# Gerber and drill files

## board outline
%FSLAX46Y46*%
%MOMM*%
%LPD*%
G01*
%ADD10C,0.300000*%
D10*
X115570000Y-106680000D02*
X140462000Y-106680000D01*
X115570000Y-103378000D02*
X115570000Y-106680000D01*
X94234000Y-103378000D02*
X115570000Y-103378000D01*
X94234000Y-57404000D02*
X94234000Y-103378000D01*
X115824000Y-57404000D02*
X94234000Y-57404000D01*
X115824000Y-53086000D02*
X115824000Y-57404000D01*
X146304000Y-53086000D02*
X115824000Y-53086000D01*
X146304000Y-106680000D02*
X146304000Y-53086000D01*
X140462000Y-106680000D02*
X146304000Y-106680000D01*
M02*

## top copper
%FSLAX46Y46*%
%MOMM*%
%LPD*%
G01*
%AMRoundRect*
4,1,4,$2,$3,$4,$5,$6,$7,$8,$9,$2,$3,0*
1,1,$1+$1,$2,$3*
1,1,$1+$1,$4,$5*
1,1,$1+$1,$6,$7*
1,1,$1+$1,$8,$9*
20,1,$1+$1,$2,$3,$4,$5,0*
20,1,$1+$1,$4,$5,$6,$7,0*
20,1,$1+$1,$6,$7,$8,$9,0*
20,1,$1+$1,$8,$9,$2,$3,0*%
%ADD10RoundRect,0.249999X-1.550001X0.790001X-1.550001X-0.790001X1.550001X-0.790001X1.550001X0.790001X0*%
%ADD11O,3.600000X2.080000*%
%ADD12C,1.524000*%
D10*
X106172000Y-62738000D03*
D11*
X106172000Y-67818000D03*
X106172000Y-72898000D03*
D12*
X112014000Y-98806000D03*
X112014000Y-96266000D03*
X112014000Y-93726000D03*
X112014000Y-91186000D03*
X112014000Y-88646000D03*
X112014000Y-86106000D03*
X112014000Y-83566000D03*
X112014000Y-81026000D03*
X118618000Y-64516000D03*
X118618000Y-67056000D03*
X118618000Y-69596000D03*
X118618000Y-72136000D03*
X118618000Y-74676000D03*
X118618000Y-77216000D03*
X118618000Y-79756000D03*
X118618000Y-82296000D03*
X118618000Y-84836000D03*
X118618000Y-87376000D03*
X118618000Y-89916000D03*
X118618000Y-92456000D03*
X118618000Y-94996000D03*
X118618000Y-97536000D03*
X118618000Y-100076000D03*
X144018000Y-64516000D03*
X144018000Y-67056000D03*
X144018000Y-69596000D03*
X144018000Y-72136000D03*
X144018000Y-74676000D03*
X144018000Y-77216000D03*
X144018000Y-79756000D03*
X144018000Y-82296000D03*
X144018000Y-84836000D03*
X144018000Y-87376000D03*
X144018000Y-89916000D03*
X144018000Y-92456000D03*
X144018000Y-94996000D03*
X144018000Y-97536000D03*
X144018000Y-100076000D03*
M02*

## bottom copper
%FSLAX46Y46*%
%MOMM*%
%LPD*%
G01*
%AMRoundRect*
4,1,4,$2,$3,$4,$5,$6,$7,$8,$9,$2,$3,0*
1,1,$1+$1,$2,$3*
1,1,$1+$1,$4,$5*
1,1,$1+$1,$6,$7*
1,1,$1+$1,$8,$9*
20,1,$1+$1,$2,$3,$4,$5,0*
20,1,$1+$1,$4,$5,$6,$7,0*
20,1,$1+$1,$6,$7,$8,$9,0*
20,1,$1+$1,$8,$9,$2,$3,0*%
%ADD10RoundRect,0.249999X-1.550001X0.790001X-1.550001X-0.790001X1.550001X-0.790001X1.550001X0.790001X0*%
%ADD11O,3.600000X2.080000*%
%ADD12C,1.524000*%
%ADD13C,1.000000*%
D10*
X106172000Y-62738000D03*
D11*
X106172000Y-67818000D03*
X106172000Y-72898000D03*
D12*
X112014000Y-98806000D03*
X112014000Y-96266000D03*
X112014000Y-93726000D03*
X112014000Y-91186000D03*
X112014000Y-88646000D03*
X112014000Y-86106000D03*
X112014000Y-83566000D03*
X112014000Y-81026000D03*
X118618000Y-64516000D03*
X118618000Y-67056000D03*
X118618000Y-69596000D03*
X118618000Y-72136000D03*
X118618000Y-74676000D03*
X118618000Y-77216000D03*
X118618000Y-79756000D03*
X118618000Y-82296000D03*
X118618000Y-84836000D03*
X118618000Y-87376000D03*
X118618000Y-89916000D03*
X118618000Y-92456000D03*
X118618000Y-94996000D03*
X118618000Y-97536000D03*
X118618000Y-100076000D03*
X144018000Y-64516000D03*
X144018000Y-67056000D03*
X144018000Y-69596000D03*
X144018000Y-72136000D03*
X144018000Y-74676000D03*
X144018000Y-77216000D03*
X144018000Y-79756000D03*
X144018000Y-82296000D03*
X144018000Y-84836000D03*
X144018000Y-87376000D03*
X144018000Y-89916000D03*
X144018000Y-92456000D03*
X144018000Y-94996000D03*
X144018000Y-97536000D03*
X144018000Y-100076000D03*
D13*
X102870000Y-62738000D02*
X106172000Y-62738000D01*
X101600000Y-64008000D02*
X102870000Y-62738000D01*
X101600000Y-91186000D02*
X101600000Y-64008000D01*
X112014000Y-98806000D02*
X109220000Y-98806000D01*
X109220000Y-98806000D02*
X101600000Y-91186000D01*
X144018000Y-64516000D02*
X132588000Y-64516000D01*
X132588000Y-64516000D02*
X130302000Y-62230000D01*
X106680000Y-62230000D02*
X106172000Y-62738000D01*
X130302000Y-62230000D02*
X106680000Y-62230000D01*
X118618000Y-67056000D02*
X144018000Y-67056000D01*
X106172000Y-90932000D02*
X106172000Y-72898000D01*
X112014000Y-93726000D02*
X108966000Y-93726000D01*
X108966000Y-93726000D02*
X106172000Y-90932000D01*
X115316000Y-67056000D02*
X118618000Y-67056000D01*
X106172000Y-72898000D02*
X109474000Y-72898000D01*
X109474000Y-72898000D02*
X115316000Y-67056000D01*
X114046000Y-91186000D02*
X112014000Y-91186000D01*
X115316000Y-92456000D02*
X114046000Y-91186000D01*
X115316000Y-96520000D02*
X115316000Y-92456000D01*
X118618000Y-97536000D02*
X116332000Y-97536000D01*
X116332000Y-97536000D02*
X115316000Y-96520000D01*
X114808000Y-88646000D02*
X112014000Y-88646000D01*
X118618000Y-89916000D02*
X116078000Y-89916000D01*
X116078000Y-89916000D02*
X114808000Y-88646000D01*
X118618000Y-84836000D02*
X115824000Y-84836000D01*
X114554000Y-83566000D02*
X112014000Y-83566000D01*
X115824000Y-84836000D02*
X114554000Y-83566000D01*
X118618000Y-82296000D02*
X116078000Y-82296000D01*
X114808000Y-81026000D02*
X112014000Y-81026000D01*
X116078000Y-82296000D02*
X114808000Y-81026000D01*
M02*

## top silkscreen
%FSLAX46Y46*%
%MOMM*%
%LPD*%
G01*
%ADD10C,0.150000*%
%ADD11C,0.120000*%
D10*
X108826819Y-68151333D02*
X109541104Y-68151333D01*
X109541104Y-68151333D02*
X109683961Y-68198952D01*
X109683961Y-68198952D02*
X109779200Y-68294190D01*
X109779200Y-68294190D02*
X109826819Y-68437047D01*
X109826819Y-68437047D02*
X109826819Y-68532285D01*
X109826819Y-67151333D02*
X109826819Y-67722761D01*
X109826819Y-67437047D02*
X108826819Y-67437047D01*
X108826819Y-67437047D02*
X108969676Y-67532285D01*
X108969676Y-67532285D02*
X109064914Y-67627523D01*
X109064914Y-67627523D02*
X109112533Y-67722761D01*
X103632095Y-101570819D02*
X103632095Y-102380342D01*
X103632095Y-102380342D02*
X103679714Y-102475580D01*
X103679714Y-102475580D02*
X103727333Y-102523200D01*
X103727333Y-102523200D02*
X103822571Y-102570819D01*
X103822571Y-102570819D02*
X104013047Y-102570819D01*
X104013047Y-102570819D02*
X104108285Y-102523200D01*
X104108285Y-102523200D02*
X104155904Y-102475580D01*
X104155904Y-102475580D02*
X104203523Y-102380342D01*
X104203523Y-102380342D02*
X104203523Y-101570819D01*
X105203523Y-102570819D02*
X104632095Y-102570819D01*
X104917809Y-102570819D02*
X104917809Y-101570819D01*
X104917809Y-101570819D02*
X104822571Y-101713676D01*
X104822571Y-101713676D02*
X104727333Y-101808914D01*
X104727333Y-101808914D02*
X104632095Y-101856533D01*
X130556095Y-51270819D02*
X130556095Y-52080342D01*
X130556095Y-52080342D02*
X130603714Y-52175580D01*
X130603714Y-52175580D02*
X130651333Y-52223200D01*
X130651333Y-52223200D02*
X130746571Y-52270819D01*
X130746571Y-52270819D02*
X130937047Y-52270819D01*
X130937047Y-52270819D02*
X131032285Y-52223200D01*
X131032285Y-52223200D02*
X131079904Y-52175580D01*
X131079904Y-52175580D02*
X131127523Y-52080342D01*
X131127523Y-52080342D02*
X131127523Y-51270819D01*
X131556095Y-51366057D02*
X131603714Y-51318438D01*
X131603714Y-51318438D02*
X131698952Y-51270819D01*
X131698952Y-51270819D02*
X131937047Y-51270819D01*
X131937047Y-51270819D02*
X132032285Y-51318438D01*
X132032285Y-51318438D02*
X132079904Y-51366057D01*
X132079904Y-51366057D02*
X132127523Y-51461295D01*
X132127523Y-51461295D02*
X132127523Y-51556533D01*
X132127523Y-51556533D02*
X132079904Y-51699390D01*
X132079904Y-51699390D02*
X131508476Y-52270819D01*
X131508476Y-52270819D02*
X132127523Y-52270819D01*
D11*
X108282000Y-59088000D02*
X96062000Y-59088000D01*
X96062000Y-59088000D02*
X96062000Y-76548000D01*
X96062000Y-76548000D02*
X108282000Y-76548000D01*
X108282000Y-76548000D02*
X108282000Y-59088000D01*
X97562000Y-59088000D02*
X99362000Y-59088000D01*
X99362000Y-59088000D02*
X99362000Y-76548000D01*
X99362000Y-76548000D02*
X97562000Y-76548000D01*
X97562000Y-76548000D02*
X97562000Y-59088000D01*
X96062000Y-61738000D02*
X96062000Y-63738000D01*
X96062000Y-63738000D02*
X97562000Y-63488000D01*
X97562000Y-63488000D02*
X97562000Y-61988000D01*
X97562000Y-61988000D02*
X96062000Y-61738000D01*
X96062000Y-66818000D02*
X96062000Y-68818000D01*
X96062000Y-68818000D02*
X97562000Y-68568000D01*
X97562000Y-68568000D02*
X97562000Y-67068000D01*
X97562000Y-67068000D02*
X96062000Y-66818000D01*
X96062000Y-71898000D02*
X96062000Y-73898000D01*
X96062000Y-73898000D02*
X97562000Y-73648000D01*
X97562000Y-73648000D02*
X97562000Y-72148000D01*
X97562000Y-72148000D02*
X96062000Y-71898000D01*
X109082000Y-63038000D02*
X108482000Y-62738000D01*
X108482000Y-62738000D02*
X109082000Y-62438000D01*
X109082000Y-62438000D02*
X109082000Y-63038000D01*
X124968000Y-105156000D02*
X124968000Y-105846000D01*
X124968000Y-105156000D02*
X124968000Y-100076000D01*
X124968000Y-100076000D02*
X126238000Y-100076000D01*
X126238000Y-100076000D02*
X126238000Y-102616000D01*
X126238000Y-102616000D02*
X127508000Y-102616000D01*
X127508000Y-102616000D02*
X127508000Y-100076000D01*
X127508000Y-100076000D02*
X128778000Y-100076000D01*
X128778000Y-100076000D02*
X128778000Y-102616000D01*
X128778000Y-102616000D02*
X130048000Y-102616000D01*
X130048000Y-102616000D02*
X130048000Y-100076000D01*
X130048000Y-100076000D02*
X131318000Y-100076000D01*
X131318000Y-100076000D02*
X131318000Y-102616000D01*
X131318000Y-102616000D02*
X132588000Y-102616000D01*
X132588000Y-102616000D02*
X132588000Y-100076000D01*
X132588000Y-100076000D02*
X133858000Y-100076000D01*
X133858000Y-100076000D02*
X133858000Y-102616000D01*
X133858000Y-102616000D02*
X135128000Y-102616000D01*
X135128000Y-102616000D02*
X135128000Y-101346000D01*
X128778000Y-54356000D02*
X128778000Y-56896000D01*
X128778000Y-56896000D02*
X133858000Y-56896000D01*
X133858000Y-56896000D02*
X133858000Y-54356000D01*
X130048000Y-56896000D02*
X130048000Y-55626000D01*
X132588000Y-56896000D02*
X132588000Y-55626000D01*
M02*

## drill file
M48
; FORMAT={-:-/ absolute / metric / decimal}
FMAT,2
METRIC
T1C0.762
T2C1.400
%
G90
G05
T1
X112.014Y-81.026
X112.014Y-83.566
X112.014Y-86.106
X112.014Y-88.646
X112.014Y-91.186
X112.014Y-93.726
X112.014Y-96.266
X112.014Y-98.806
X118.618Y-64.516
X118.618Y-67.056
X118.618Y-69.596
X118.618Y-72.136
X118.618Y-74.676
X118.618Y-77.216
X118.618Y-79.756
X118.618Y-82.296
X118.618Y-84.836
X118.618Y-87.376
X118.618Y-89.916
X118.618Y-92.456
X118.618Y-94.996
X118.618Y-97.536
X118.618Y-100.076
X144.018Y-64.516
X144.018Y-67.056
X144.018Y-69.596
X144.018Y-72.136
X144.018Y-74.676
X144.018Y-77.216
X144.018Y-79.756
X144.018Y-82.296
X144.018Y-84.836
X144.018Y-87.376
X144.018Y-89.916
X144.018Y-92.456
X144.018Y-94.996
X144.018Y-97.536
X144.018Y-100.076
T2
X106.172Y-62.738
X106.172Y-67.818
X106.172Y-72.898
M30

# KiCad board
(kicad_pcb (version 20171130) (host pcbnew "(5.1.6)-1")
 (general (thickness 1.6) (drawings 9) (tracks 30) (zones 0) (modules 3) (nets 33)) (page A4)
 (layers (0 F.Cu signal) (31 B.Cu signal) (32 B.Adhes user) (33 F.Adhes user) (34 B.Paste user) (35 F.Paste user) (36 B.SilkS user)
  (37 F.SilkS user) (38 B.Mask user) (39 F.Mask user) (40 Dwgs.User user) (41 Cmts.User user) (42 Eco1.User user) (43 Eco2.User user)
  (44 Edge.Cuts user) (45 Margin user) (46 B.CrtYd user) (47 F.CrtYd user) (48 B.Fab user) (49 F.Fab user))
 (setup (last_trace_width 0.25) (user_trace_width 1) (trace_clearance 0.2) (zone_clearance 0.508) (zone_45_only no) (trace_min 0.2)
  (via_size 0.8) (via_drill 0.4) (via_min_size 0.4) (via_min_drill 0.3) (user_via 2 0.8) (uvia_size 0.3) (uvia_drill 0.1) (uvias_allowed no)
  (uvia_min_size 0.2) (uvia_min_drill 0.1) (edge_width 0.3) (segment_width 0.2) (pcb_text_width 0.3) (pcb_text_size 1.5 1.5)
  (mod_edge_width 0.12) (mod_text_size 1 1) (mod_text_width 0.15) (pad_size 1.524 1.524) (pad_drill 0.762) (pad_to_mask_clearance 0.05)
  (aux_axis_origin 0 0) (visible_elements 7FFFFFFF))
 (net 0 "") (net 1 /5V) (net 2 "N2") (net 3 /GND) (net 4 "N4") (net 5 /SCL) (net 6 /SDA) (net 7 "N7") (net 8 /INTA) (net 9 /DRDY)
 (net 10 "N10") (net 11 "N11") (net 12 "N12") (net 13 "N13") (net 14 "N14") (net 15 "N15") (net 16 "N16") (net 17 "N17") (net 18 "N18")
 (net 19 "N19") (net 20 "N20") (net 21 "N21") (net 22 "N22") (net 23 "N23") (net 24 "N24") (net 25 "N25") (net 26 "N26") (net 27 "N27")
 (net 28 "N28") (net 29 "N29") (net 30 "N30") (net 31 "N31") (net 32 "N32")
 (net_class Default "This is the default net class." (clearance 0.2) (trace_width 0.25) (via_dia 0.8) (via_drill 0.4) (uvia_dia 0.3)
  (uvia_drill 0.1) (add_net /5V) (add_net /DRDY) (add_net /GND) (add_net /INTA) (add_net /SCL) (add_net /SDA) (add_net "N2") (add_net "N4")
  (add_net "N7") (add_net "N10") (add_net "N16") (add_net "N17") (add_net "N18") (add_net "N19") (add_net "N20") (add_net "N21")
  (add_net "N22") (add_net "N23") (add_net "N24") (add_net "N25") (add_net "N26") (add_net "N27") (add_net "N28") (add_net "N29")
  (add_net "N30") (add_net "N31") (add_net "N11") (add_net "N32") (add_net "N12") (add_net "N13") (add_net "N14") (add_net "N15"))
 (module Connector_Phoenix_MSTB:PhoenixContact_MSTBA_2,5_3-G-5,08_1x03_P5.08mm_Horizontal (layer F.Cu) (at 106.172 62.738 270)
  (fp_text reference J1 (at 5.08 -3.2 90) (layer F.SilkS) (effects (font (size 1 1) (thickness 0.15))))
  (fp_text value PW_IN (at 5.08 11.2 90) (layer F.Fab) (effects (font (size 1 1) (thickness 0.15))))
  (fp_line (start -3.65 -2.11) (end -3.65 10.11) (layer F.SilkS) (width 0.12))
  (fp_line (start -3.65 10.11) (end 13.81 10.11) (layer F.SilkS) (width 0.12))
  (fp_line (start 13.81 10.11) (end 13.81 -2.11) (layer F.SilkS) (width 0.12))
  (fp_line (start 13.81 -2.11) (end -3.65 -2.11) (layer F.SilkS) (width 0.12))
  (fp_line (start -3.65 8.61) (end -3.65 6.81) (layer F.SilkS) (width 0.12))
  (fp_line (start -3.65 6.81) (end 13.81 6.81) (layer F.SilkS) (width 0.12))
  (fp_line (start 13.81 6.81) (end 13.81 8.61) (layer F.SilkS) (width 0.12))
  (fp_line (start 13.81 8.61) (end -3.65 8.61) (layer F.SilkS) (width 0.12))
  (fp_line (start -1 10.11) (end 1 10.11) (layer F.SilkS) (width 0.12))
  (fp_line (start 1 10.11) (end 0.75 8.61) (layer F.SilkS) (width 0.12))
  (fp_line (start 0.75 8.61) (end -0.75 8.61) (layer F.SilkS) (width 0.12))
  (fp_line (start -0.75 8.61) (end -1 10.11) (layer F.SilkS) (width 0.12))
  (fp_line (start 4.08 10.11) (end 6.08 10.11) (layer F.SilkS) (width 0.12))
  (fp_line (start 6.08 10.11) (end 5.83 8.61) (layer F.SilkS) (width 0.12))
  (fp_line (start 5.83 8.61) (end 4.33 8.61) (layer F.SilkS) (width 0.12))
  (fp_line (start 4.33 8.61) (end 4.08 10.11) (layer F.SilkS) (width 0.12))
  (fp_line (start 9.16 10.11) (end 11.16 10.11) (layer F.SilkS) (width 0.12))
  (fp_line (start 11.16 10.11) (end 10.91 8.61) (layer F.SilkS) (width 0.12))
  (fp_line (start 10.91 8.61) (end 9.41 8.61) (layer F.SilkS) (width 0.12))
  (fp_line (start 9.41 8.61) (end 9.16 10.11) (layer F.SilkS) (width 0.12))
  (fp_line (start 0.3 -2.91) (end 0 -2.31) (layer F.SilkS) (width 0.12))
  (fp_line (start 0 -2.31) (end -0.3 -2.91) (layer F.SilkS) (width 0.12))
  (fp_line (start -0.3 -2.91) (end 0.3 -2.91) (layer F.SilkS) (width 0.12))
  (pad 1 thru_hole roundrect (at 0 0 270) (size 2.08 3.6) (drill 1.4) (layers *.Cu *.Mask) (roundrect_rratio 0.120192) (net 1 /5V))
  (pad 2 thru_hole oval (at 5.08 0 270) (size 2.08 3.6) (drill 1.4) (layers *.Cu *.Mask) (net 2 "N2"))
  (pad 3 thru_hole oval (at 10.16 0 270) (size 2.08 3.6) (drill 1.4) (layers *.Cu *.Mask) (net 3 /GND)))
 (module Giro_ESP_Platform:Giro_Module (layer F.Cu) (at 112.014 102.616 180)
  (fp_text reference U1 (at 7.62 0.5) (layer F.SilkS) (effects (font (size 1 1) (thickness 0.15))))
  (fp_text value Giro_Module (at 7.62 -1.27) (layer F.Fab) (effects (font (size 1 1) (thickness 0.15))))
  (pad 1 thru_hole circle (at 0 3.81 180) (size 1.524 1.524) (drill 0.762) (layers *.Cu *.Mask) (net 1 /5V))
  (pad 2 thru_hole circle (at 0 6.35 180) (size 1.524 1.524) (drill 0.762) (layers *.Cu *.Mask) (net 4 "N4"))
  (pad 3 thru_hole circle (at 0 8.89 180) (size 1.524 1.524) (drill 0.762) (layers *.Cu *.Mask) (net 3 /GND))
  (pad 4 thru_hole circle (at 0 11.43 180) (size 1.524 1.524) (drill 0.762) (layers *.Cu *.Mask) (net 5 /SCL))
  (pad 5 thru_hole circle (at 0 13.97 180) (size 1.524 1.524) (drill 0.762) (layers *.Cu *.Mask) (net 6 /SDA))
  (pad 6 thru_hole circle (at 0 16.51 180) (size 1.524 1.524) (drill 0.762) (layers *.Cu *.Mask) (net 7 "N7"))
  (pad 7 thru_hole circle (at 0 19.05 180) (size 1.524 1.524) (drill 0.762) (layers *.Cu *.Mask) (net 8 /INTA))
  (pad 8 thru_hole circle (at 0 21.59 180) (size 1.524 1.524) (drill 0.762) (layers *.Cu *.Mask) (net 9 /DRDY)))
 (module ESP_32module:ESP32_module (layer F.Cu) (at 124.968 74.676)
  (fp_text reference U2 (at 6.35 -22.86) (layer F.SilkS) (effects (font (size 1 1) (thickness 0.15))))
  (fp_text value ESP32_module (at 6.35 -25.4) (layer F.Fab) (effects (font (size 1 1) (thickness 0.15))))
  (fp_line (start 0 30.48) (end 0 31.17) (layer F.SilkS) (width 0.12))
  (fp_line (start 0 30.48) (end 0 25.4) (layer F.SilkS) (width 0.12))
  (fp_line (start 0 25.4) (end 1.27 25.4) (layer F.SilkS) (width 0.12))
  (fp_line (start 1.27 25.4) (end 1.27 27.94) (layer F.SilkS) (width 0.12))
  (fp_line (start 1.27 27.94) (end 2.54 27.94) (layer F.SilkS) (width 0.12))
  (fp_line (start 2.54 27.94) (end 2.54 25.4) (layer F.SilkS) (width 0.12))
  (fp_line (start 2.54 25.4) (end 3.81 25.4) (layer F.SilkS) (width 0.12))
  (fp_line (start 3.81 25.4) (end 3.81 27.94) (layer F.SilkS) (width 0.12))
  (fp_line (start 3.81 27.94) (end 5.08 27.94) (layer F.SilkS) (width 0.12))
  (fp_line (start 5.08 27.94) (end 5.08 25.4) (layer F.SilkS) (width 0.12))
  (fp_line (start 5.08 25.4) (end 6.35 25.4) (layer F.SilkS) (width 0.12))
  (fp_line (start 6.35 25.4) (end 6.35 27.94) (layer F.SilkS) (width 0.12))
  (fp_line (start 6.35 27.94) (end 7.62 27.94) (layer F.SilkS) (width 0.12))
  (fp_line (start 7.62 27.94) (end 7.62 25.4) (layer F.SilkS) (width 0.12))
  (fp_line (start 7.62 25.4) (end 8.89 25.4) (layer F.SilkS) (width 0.12))
  (fp_line (start 8.89 25.4) (end 8.89 27.94) (layer F.SilkS) (width 0.12))
  (fp_line (start 8.89 27.94) (end 10.16 27.94) (layer F.SilkS) (width 0.12))
  (fp_line (start 10.16 27.94) (end 10.16 26.67) (layer F.SilkS) (width 0.12))
  (fp_line (start 3.81 -20.32) (end 3.81 -17.78) (layer F.SilkS) (width 0.12))
  (fp_line (start 3.81 -17.78) (end 8.89 -17.78) (layer F.SilkS) (width 0.12))
  (fp_line (start 8.89 -17.78) (end 8.89 -20.32) (layer F.SilkS) (width 0.12))
  (fp_line (start 5.08 -17.78) (end 5.08 -19.05) (layer F.SilkS) (width 0.12))
  (fp_line (start 7.62 -17.78) (end 7.62 -19.05) (layer F.SilkS) (width 0.12))
  (pad 1 thru_hole circle (at -6.35 -10.16) (size 1.524 1.524) (drill 0.762) (layers *.Cu *.Mask) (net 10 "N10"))
  (pad 2 thru_hole circle (at -6.35 -7.62) (size 1.524 1.524) (drill 0.762) (layers *.Cu *.Mask) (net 3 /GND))
  (pad 3 thru_hole circle (at -6.35 -5.08) (size 1.524 1.524) (drill 0.762) (layers *.Cu *.Mask) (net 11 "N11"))
  (pad 4 thru_hole circle (at -6.35 -2.54) (size 1.524 1.524) (drill 0.762) (layers *.Cu *.Mask) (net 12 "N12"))
  (pad 5 thru_hole circle (at -6.35 0) (size 1.524 1.524) (drill 0.762) (layers *.Cu *.Mask) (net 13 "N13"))
  (pad 6 thru_hole circle (at -6.35 2.54) (size 1.524 1.524) (drill 0.762) (layers *.Cu *.Mask) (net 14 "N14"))
  (pad 7 thru_hole circle (at -6.35 5.08) (size 1.524 1.524) (drill 0.762) (layers *.Cu *.Mask) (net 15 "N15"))
  (pad 8 thru_hole circle (at -6.35 7.62) (size 1.524 1.524) (drill 0.762) (layers *.Cu *.Mask) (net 9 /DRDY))
  (pad 9 thru_hole circle (at -6.35 10.16) (size 1.524 1.524) (drill 0.762) (layers *.Cu *.Mask) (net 8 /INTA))
  (pad 10 thru_hole circle (at -6.35 12.7) (size 1.524 1.524) (drill 0.762) (layers *.Cu *.Mask) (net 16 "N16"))
  (pad 11 thru_hole circle (at -6.35 15.24) (size 1.524 1.524) (drill 0.762) (layers *.Cu *.Mask) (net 6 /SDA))
  (pad 12 thru_hole circle (at -6.35 17.78) (size 1.524 1.524) (drill 0.762) (layers *.Cu *.Mask) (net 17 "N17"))
  (pad 13 thru_hole circle (at -6.35 20.32) (size 1.524 1.524) (drill 0.762) (layers *.Cu *.Mask) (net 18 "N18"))
  (pad 14 thru_hole circle (at -6.35 22.86) (size 1.524 1.524) (drill 0.762) (layers *.Cu *.Mask) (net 5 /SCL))
  (pad 15 thru_hole circle (at -6.35 25.4) (size 1.524 1.524) (drill 0.762) (layers *.Cu *.Mask) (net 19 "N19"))
  (pad 16 thru_hole circle (at 19.05 -10.16) (size 1.524 1.524) (drill 0.762) (layers *.Cu *.Mask) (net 1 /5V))
  (pad 17 thru_hole circle (at 19.05 -7.62) (size 1.524 1.524) (drill 0.762) (layers *.Cu *.Mask) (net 3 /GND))
  (pad 18 thru_hole circle (at 19.05 -5.08) (size 1.524 1.524) (drill 0.762) (layers *.Cu *.Mask) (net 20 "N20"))
  (pad 19 thru_hole circle (at 19.05 -2.54) (size 1.524 1.524) (drill 0.762) (layers *.Cu *.Mask) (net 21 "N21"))
  (pad 20 thru_hole circle (at 19.05 0) (size 1.524 1.524) (drill 0.762) (layers *.Cu *.Mask) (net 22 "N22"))
  (pad 21 thru_hole circle (at 19.05 2.54) (size 1.524 1.524) (drill 0.762) (layers *.Cu *.Mask) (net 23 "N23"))
  (pad 22 thru_hole circle (at 19.05 5.08) (size 1.524 1.524) (drill 0.762) (layers *.Cu *.Mask) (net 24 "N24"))
  (pad 23 thru_hole circle (at 19.05 7.62) (size 1.524 1.524) (drill 0.762) (layers *.Cu *.Mask) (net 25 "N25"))
  (pad 24 thru_hole circle (at 19.05 10.16) (size 1.524 1.524) (drill 0.762) (layers *.Cu *.Mask) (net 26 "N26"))
  (pad 25 thru_hole circle (at 19.05 12.7) (size 1.524 1.524) (drill 0.762) (layers *.Cu *.Mask) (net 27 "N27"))
  (pad 26 thru_hole circle (at 19.05 15.24) (size 1.524 1.524) (drill 0.762) (layers *.Cu *.Mask) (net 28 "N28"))
  (pad 27 thru_hole circle (at 19.05 17.78) (size 1.524 1.524) (drill 0.762) (layers *.Cu *.Mask) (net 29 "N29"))
  (pad 28 thru_hole circle (at 19.05 20.32) (size 1.524 1.524) (drill 0.762) (layers *.Cu *.Mask) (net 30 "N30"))
  (pad 29 thru_hole circle (at 19.05 22.86) (size 1.524 1.524) (drill 0.762) (layers *.Cu *.Mask) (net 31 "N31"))
  (pad 30 thru_hole circle (at 19.05 25.4) (size 1.524 1.524) (drill 0.762) (layers *.Cu *.Mask) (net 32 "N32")))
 (gr_line (start 115.57 106.68) (end 140.462 106.68) (layer Edge.Cuts) (width 0.3))
 (gr_line (start 115.57 103.378) (end 115.57 106.68) (layer Edge.Cuts) (width 0.3))
 (gr_line (start 94.234 103.378) (end 115.57 103.378) (layer Edge.Cuts) (width 0.3))
 (gr_line (start 94.234 57.404) (end 94.234 103.378) (layer Edge.Cuts) (width 0.3))
 (gr_line (start 115.824 57.404) (end 94.234 57.404) (layer Edge.Cuts) (width 0.3))
 (gr_line (start 115.824 53.086) (end 115.824 57.404) (layer Edge.Cuts) (width 0.3))
 (gr_line (start 146.304 53.086) (end 115.824 53.086) (layer Edge.Cuts) (width 0.3))
 (gr_line (start 146.304 106.68) (end 146.304 53.086) (layer Edge.Cuts) (width 0.3))
 (gr_line (start 140.462 106.68) (end 146.304 106.68) (layer Edge.Cuts) (width 0.3))
 (segment (start 102.87 62.738) (end 106.172 62.738) (width 1) (layer B.Cu) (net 1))
 (segment (start 101.6 64.008) (end 102.87 62.738) (width 1) (layer B.Cu) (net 1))
 (segment (start 101.6 91.186) (end 101.6 64.008) (width 1) (layer B.Cu) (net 1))
 (segment (start 112.014 98.806) (end 109.22 98.806) (width 1) (layer B.Cu) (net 1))
 (segment (start 109.22 98.806) (end 101.6 91.186) (width 1) (layer B.Cu) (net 1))
 (segment (start 144.018 64.516) (end 132.588 64.516) (width 1) (layer B.Cu) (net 1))
 (segment (start 132.588 64.516) (end 130.302 62.23) (width 1) (layer B.Cu) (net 1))
 (segment (start 106.68 62.23) (end 106.172 62.738) (width 1) (layer B.Cu) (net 1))
 (segment (start 130.302 62.23) (end 106.68 62.23) (width 1) (layer B.Cu) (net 1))
 (segment (start 118.618 67.056) (end 144.018 67.056) (width 1) (layer B.Cu) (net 3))
 (segment (start 106.172 90.932) (end 106.172 72.898) (width 1) (layer B.Cu) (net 3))
 (segment (start 112.014 93.726) (end 108.966 93.726) (width 1) (layer B.Cu) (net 3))
 (segment (start 108.966 93.726) (end 106.172 90.932) (width 1) (layer B.Cu) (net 3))
 (segment (start 115.316 67.056) (end 118.618 67.056) (width 1) (layer B.Cu) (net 3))
 (segment (start 106.172 72.898) (end 109.474 72.898) (width 1) (layer B.Cu) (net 3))
 (segment (start 109.474 72.898) (end 115.316 67.056) (width 1) (layer B.Cu) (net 3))
 (segment (start 114.046 91.186) (end 112.014 91.186) (width 1) (layer B.Cu) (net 5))
 (segment (start 115.316 92.456) (end 114.046 91.186) (width 1) (layer B.Cu) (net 5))
 (segment (start 115.316 96.52) (end 115.316 92.456) (width 1) (layer B.Cu) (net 5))
 (segment (start 118.618 97.536) (end 116.332 97.536) (width 1) (layer B.Cu) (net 5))
 (segment (start 116.332 97.536) (end 115.316 96.52) (width 1) (layer B.Cu) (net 5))
 (segment (start 114.808 88.646) (end 112.014 88.646) (width 1) (layer B.Cu) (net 6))
 (segment (start 118.618 89.916) (end 116.078 89.916) (width 1) (layer B.Cu) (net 6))
 (segment (start 116.078 89.916) (end 114.808 88.646) (width 1) (layer B.Cu) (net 6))
 (segment (start 118.618 84.836) (end 115.824 84.836) (width 1) (layer B.Cu) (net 8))
 (segment (start 114.554 83.566) (end 112.014 83.566) (width 1) (layer B.Cu) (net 8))
 (segment (start 115.824 84.836) (end 114.554 83.566) (width 1) (layer B.Cu) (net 8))
 (segment (start 118.618 82.296) (end 116.078 82.296) (width 1) (layer B.Cu) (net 9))
 (segment (start 114.808 81.026) (end 112.014 81.026) (width 1) (layer B.Cu) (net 9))
 (segment (start 116.078 82.296) (end 114.808 81.026) (width 1) (layer B.Cu) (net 9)))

